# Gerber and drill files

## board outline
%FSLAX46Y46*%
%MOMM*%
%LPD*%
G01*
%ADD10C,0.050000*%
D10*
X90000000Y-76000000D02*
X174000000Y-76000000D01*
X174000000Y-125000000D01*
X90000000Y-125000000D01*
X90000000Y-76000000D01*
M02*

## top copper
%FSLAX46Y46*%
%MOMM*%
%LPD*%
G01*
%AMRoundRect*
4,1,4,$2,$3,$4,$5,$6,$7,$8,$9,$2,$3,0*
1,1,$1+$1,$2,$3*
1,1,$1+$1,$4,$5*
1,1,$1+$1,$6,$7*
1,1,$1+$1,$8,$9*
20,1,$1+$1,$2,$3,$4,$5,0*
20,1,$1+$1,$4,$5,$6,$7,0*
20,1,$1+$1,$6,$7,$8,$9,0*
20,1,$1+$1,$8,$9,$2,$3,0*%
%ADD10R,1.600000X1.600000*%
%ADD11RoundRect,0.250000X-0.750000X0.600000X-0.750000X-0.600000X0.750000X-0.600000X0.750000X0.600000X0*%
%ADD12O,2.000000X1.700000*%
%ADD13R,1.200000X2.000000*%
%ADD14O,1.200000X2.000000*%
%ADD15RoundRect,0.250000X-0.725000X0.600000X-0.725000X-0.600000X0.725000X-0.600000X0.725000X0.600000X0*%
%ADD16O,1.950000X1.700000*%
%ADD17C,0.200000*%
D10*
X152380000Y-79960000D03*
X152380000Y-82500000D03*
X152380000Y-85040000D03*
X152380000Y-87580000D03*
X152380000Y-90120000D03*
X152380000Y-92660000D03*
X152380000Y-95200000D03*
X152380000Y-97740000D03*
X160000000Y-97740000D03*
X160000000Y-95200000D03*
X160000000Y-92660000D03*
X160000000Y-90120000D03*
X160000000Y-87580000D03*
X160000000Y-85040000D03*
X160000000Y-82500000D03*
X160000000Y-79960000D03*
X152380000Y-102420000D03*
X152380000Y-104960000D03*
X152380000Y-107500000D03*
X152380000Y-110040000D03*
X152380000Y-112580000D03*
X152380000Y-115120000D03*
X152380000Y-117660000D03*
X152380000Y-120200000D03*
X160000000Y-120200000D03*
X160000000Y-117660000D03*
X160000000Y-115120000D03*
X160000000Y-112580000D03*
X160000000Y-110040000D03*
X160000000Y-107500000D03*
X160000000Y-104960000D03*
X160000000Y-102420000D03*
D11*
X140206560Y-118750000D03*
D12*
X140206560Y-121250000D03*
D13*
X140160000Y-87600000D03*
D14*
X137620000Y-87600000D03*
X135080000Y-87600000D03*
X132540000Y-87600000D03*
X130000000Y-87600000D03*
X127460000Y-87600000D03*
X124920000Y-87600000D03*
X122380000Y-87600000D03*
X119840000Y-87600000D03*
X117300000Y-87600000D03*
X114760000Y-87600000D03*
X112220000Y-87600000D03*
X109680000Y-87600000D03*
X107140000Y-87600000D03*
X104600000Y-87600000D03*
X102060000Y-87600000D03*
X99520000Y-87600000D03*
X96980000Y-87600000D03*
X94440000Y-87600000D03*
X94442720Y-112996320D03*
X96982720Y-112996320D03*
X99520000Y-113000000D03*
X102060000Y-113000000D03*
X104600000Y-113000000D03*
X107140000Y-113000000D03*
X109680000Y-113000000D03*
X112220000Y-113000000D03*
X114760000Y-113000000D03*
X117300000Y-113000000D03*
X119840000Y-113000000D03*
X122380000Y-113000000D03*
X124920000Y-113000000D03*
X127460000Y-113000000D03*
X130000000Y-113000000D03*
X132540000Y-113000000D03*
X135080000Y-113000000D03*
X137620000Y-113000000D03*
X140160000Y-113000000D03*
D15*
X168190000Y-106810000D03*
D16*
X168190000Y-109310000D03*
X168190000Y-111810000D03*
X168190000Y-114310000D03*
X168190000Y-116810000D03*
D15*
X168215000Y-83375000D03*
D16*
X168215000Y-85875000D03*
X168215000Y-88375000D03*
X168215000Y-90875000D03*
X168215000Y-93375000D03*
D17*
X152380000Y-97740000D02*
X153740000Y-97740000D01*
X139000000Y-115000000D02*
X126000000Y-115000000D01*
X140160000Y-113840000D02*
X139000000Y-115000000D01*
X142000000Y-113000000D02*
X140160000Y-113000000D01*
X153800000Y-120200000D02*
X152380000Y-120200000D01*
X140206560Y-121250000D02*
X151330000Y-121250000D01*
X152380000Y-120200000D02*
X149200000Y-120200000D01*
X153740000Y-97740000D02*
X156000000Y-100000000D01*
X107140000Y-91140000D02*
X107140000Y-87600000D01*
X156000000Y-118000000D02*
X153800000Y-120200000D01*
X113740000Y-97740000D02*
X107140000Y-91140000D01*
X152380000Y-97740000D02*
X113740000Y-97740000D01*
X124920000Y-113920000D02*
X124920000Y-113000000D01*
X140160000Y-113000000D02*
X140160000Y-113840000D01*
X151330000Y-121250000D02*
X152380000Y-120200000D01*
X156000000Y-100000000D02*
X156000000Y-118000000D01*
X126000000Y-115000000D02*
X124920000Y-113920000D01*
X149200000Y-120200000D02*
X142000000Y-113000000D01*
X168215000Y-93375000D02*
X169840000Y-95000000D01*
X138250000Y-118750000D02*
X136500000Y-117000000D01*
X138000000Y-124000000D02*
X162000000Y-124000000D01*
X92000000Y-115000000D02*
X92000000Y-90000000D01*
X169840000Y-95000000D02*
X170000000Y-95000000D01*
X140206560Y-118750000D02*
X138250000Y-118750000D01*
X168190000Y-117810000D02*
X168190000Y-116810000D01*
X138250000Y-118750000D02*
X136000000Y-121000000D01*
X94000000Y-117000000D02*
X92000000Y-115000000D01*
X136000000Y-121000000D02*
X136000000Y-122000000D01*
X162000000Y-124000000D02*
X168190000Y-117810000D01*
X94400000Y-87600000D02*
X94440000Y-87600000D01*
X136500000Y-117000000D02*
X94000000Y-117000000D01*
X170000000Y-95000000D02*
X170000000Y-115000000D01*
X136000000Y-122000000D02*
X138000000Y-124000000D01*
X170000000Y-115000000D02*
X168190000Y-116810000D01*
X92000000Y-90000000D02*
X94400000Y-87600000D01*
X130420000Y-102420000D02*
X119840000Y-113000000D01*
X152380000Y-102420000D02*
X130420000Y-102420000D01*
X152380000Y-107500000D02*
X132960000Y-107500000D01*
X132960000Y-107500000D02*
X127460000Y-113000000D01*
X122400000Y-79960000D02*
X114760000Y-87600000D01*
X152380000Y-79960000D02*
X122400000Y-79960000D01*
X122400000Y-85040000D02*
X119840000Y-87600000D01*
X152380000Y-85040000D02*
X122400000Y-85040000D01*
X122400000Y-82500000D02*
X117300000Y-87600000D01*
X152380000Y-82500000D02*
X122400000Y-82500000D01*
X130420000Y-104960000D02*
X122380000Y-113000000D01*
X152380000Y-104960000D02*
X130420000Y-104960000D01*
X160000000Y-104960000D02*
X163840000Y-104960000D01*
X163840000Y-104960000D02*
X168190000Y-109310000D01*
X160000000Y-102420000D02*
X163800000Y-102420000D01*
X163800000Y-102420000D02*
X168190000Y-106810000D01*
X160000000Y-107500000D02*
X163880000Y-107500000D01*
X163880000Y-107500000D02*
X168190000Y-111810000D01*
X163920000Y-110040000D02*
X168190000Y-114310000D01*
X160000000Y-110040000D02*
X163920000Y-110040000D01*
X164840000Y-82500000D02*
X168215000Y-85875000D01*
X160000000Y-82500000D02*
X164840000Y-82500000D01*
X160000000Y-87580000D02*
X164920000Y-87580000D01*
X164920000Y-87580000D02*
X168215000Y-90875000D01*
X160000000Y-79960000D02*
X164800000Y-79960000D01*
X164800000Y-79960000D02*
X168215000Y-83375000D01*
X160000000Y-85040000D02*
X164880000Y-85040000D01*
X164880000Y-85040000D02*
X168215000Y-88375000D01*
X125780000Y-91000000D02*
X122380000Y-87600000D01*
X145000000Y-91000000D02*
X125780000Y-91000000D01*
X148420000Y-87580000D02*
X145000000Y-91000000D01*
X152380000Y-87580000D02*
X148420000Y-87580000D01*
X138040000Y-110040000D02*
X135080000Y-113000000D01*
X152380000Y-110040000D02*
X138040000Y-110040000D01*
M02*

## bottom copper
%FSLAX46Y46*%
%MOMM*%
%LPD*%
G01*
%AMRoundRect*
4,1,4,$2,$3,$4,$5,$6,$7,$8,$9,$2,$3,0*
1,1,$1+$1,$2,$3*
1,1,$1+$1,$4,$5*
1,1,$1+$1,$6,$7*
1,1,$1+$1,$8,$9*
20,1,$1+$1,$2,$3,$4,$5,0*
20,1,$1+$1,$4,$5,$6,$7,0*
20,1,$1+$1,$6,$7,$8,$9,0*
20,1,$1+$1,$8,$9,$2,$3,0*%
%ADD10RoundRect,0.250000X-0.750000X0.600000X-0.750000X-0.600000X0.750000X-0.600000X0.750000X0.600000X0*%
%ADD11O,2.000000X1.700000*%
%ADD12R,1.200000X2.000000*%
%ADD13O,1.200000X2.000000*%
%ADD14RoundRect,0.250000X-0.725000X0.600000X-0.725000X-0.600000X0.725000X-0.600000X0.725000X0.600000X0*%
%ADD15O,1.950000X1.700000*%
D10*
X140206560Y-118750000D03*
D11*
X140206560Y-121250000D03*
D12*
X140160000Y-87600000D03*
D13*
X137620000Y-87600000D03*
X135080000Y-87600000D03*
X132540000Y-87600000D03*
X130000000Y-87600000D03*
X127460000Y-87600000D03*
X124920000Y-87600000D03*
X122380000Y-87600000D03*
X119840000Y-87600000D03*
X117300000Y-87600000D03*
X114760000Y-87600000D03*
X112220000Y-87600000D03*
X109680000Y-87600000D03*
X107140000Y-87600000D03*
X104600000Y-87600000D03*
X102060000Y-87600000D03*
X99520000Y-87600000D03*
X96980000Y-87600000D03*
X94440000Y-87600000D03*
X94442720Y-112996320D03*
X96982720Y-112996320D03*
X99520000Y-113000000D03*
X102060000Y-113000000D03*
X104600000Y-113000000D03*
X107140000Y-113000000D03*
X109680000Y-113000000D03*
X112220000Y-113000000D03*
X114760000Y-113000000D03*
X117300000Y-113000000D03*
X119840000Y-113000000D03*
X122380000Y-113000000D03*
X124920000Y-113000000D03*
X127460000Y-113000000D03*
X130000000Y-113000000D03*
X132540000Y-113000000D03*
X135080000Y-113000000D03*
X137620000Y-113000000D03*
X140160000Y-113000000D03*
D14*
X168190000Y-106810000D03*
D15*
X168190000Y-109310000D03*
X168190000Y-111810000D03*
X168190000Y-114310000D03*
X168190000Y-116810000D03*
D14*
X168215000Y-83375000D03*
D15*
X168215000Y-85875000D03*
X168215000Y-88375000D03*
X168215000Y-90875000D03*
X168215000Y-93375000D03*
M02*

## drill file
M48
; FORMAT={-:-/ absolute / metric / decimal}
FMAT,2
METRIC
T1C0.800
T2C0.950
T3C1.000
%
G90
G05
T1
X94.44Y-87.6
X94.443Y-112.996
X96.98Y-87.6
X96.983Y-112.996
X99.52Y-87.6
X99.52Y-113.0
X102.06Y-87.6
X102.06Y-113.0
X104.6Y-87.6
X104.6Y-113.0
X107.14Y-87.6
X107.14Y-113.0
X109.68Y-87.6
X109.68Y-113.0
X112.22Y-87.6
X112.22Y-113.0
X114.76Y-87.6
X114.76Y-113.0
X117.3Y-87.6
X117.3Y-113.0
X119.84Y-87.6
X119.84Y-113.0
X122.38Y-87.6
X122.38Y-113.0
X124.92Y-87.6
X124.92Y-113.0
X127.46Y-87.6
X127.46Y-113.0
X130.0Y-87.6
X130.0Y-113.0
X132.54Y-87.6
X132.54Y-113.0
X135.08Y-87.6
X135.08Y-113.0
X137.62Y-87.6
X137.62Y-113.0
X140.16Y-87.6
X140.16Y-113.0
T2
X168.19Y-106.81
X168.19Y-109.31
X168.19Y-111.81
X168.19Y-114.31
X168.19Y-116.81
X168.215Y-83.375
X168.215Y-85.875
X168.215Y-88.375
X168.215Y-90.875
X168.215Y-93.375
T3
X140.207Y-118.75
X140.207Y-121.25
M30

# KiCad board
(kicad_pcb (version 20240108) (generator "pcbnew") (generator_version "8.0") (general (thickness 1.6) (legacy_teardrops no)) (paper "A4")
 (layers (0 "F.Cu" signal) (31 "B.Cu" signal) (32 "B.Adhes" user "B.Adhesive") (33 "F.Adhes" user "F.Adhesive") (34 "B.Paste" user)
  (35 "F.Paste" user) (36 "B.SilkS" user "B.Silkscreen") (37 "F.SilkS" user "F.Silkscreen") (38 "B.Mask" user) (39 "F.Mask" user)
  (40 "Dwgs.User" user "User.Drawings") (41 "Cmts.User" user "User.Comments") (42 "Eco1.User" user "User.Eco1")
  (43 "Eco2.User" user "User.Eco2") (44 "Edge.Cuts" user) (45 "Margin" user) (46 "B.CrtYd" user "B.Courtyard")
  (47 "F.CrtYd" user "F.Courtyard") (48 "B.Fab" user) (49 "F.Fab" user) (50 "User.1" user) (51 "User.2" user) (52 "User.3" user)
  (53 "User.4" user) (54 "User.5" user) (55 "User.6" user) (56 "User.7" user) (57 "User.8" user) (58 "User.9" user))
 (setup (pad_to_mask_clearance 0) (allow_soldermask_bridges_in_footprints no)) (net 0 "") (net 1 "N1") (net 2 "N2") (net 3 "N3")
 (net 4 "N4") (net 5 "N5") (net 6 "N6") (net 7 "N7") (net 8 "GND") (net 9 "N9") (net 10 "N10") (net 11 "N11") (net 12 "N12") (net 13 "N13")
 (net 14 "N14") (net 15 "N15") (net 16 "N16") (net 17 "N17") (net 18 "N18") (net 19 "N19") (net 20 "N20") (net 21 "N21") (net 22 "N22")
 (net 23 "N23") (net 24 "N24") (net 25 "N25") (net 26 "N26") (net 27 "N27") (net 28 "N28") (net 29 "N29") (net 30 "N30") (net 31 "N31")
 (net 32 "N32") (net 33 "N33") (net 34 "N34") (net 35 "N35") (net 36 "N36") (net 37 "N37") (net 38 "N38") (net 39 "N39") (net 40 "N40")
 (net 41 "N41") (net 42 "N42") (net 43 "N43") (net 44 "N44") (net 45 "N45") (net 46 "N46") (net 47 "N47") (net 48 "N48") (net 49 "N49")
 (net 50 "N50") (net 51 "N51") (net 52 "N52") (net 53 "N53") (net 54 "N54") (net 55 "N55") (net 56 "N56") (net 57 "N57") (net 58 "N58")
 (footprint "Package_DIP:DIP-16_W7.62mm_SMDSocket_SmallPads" (layer "F.Cu") (at 156.19 88.85)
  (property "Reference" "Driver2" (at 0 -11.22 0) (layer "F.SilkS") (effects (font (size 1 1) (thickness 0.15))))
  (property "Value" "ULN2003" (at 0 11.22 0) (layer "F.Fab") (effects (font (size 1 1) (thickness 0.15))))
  (pad "1" smd rect (at -3.81 -8.89) (size 1.6 1.6) (layers "F.Cu" "F.Paste" "F.Mask") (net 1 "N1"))
  (pad "2" smd rect (at -3.81 -6.35) (size 1.6 1.6) (layers "F.Cu" "F.Paste" "F.Mask") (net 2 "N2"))
  (pad "3" smd rect (at -3.81 -3.81) (size 1.6 1.6) (layers "F.Cu" "F.Paste" "F.Mask") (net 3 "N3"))
  (pad "4" smd rect (at -3.81 -1.27) (size 1.6 1.6) (layers "F.Cu" "F.Paste" "F.Mask") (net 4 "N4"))
  (pad "5" smd rect (at -3.81 1.27) (size 1.6 1.6) (layers "F.Cu" "F.Paste" "F.Mask") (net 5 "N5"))
  (pad "6" smd rect (at -3.81 3.81) (size 1.6 1.6) (layers "F.Cu" "F.Paste" "F.Mask") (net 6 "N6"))
  (pad "7" smd rect (at -3.81 6.35) (size 1.6 1.6) (layers "F.Cu" "F.Paste" "F.Mask") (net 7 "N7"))
  (pad "8" smd rect (at -3.81 8.89) (size 1.6 1.6) (layers "F.Cu" "F.Paste" "F.Mask") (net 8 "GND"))
  (pad "9" smd rect (at 3.81 8.89) (size 1.6 1.6) (layers "F.Cu" "F.Paste" "F.Mask") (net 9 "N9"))
  (pad "10" smd rect (at 3.81 6.35) (size 1.6 1.6) (layers "F.Cu" "F.Paste" "F.Mask") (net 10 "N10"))
  (pad "11" smd rect (at 3.81 3.81) (size 1.6 1.6) (layers "F.Cu" "F.Paste" "F.Mask") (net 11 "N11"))
  (pad "12" smd rect (at 3.81 1.27) (size 1.6 1.6) (layers "F.Cu" "F.Paste" "F.Mask") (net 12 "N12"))
  (pad "13" smd rect (at 3.81 -1.27) (size 1.6 1.6) (layers "F.Cu" "F.Paste" "F.Mask") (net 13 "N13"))
  (pad "14" smd rect (at 3.81 -3.81) (size 1.6 1.6) (layers "F.Cu" "F.Paste" "F.Mask") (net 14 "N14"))
  (pad "15" smd rect (at 3.81 -6.35) (size 1.6 1.6) (layers "F.Cu" "F.Paste" "F.Mask") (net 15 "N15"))
  (pad "16" smd rect (at 3.81 -8.89) (size 1.6 1.6) (layers "F.Cu" "F.Paste" "F.Mask") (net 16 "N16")))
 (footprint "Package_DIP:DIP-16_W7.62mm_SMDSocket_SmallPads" (layer "F.Cu") (at 156.19 111.31)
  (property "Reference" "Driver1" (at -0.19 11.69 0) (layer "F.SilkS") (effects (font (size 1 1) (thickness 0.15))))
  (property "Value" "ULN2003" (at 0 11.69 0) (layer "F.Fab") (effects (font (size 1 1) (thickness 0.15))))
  (pad "1" smd rect (at -3.81 -8.89) (size 1.6 1.6) (layers "F.Cu" "F.Paste" "F.Mask") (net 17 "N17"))
  (pad "2" smd rect (at -3.81 -6.35) (size 1.6 1.6) (layers "F.Cu" "F.Paste" "F.Mask") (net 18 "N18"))
  (pad "3" smd rect (at -3.81 -3.81) (size 1.6 1.6) (layers "F.Cu" "F.Paste" "F.Mask") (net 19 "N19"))
  (pad "4" smd rect (at -3.81 -1.27) (size 1.6 1.6) (layers "F.Cu" "F.Paste" "F.Mask") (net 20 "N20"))
  (pad "5" smd rect (at -3.81 1.27) (size 1.6 1.6) (layers "F.Cu" "F.Paste" "F.Mask") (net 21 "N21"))
  (pad "6" smd rect (at -3.81 3.81) (size 1.6 1.6) (layers "F.Cu" "F.Paste" "F.Mask") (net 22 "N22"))
  (pad "7" smd rect (at -3.81 6.35) (size 1.6 1.6) (layers "F.Cu" "F.Paste" "F.Mask") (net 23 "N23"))
  (pad "8" smd rect (at -3.81 8.89) (size 1.6 1.6) (layers "F.Cu" "F.Paste" "F.Mask") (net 8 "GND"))
  (pad "9" smd rect (at 3.81 8.89) (size 1.6 1.6) (layers "F.Cu" "F.Paste" "F.Mask") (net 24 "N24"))
  (pad "10" smd rect (at 3.81 6.35) (size 1.6 1.6) (layers "F.Cu" "F.Paste" "F.Mask") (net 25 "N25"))
  (pad "11" smd rect (at 3.81 3.81) (size 1.6 1.6) (layers "F.Cu" "F.Paste" "F.Mask") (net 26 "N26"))
  (pad "12" smd rect (at 3.81 1.27) (size 1.6 1.6) (layers "F.Cu" "F.Paste" "F.Mask") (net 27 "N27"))
  (pad "13" smd rect (at 3.81 -1.27) (size 1.6 1.6) (layers "F.Cu" "F.Paste" "F.Mask") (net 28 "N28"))
  (pad "14" smd rect (at 3.81 -3.81) (size 1.6 1.6) (layers "F.Cu" "F.Paste" "F.Mask") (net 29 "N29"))
  (pad "15" smd rect (at 3.81 -6.35) (size 1.6 1.6) (layers "F.Cu" "F.Paste" "F.Mask") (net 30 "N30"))
  (pad "16" smd rect (at 3.81 -8.89) (size 1.6 1.6) (layers "F.Cu" "F.Paste" "F.Mask") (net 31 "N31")))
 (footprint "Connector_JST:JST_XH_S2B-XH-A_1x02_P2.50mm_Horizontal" (layer "F.Cu") (at 140.20656 118.75 -90)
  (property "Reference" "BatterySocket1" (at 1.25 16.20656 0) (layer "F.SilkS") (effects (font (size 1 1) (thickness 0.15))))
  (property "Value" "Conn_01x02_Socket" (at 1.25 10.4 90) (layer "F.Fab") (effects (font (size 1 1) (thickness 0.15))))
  (pad "1" thru_hole roundrect (at 0 0 270) (size 1.7 2) (drill 1) (layers "*.Cu" "*.Mask") (remove_unused_layers no)
   (roundrect_rratio 0.147059) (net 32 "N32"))
  (pad "2" thru_hole oval (at 2.5 0 270) (size 1.7 2) (drill 1) (layers "*.Cu" "*.Mask") (remove_unused_layers no) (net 8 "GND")))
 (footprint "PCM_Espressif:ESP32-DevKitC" (layer "F.Cu") (at 140.16 87.6 -90)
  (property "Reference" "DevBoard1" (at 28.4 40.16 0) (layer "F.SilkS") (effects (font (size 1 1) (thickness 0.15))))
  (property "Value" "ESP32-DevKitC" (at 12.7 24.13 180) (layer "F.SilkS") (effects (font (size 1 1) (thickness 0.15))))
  (pad "1" thru_hole rect (at 0 0 180) (size 1.2 2) (drill 0.8) (layers "*.Cu" "*.Mask") (remove_unused_layers no) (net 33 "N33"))
  (pad "2" thru_hole oval (at 0 2.54 180) (size 1.2 2) (drill 0.8) (layers "*.Cu" "*.Mask") (remove_unused_layers no) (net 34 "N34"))
  (pad "3" thru_hole oval (at 0 5.08 180) (size 1.2 2) (drill 0.8) (layers "*.Cu" "*.Mask") (remove_unused_layers no) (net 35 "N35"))
  (pad "4" thru_hole oval (at 0 7.62 180) (size 1.2 2) (drill 0.8) (layers "*.Cu" "*.Mask") (remove_unused_layers no) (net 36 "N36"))
  (pad "5" thru_hole oval (at 0 10.16 180) (size 1.2 2) (drill 0.8) (layers "*.Cu" "*.Mask") (remove_unused_layers no) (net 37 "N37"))
  (pad "6" thru_hole oval (at 0 12.7 180) (size 1.2 2) (drill 0.8) (layers "*.Cu" "*.Mask") (remove_unused_layers no) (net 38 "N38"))
  (pad "7" thru_hole oval (at 0 15.24 180) (size 1.2 2) (drill 0.8) (layers "*.Cu" "*.Mask") (remove_unused_layers no) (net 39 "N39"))
  (pad "8" thru_hole oval (at 0 17.78 180) (size 1.2 2) (drill 0.8) (layers "*.Cu" "*.Mask") (remove_unused_layers no) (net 4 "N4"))
  (pad "9" thru_hole oval (at 0 20.32 180) (size 1.2 2) (drill 0.8) (layers "*.Cu" "*.Mask") (remove_unused_layers no) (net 3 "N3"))
  (pad "10" thru_hole oval (at 0 22.86 180) (size 1.2 2) (drill 0.8) (layers "*.Cu" "*.Mask") (remove_unused_layers no) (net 2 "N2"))
  (pad "11" thru_hole oval (at 0 25.4 180) (size 1.2 2) (drill 0.8) (layers "*.Cu" "*.Mask") (remove_unused_layers no) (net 1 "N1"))
  (pad "12" thru_hole oval (at 0 27.94 180) (size 1.2 2) (drill 0.8) (layers "*.Cu" "*.Mask") (remove_unused_layers no) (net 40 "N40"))
  (pad "13" thru_hole oval (at 0 30.48 180) (size 1.2 2) (drill 0.8) (layers "*.Cu" "*.Mask") (remove_unused_layers no) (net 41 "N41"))
  (pad "14" thru_hole oval (at 0 33.02 180) (size 1.2 2) (drill 0.8) (layers "*.Cu" "*.Mask") (remove_unused_layers no) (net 8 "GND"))
  (pad "15" thru_hole oval (at 0 35.56 180) (size 1.2 2) (drill 0.8) (layers "*.Cu" "*.Mask") (remove_unused_layers no) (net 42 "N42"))
  (pad "16" thru_hole oval (at 0 38.1 180) (size 1.2 2) (drill 0.8) (layers "*.Cu" "*.Mask") (remove_unused_layers no) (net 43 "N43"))
  (pad "17" thru_hole oval (at 0 40.64 180) (size 1.2 2) (drill 0.8) (layers "*.Cu" "*.Mask") (remove_unused_layers no) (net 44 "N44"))
  (pad "18" thru_hole oval (at 0 43.18 180) (size 1.2 2) (drill 0.8) (layers "*.Cu" "*.Mask") (remove_unused_layers no) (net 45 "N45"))
  (pad "19" thru_hole oval (at 0 45.72 180) (size 1.2 2) (drill 0.8) (layers "*.Cu" "*.Mask") (remove_unused_layers no) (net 32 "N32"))
  (pad "20" thru_hole oval (at 25.39632 45.71728 180) (size 1.2 2) (drill 0.8) (layers "*.Cu" "*.Mask") (remove_unused_layers no)
   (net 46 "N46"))
  (pad "21" thru_hole oval (at 25.39632 43.17728 180) (size 1.2 2) (drill 0.8) (layers "*.Cu" "*.Mask") (remove_unused_layers no)
   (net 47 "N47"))
  (pad "22" thru_hole oval (at 25.4 40.64 180) (size 1.2 2) (drill 0.8) (layers "*.Cu" "*.Mask") (remove_unused_layers no) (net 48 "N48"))
  (pad "23" thru_hole oval (at 25.4 38.1 180) (size 1.2 2) (drill 0.8) (layers "*.Cu" "*.Mask") (remove_unused_layers no) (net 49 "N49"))
  (pad "24" thru_hole oval (at 25.4 35.56 180) (size 1.2 2) (drill 0.8) (layers "*.Cu" "*.Mask") (remove_unused_layers no) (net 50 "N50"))
  (pad "25" thru_hole oval (at 25.4 33.02 180) (size 1.2 2) (drill 0.8) (layers "*.Cu" "*.Mask") (remove_unused_layers no) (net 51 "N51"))
  (pad "26" thru_hole oval (at 25.4 30.48 180) (size 1.2 2) (drill 0.8) (layers "*.Cu" "*.Mask") (remove_unused_layers no) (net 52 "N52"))
  (pad "27" thru_hole oval (at 25.4 27.94 180) (size 1.2 2) (drill 0.8) (layers "*.Cu" "*.Mask") (remove_unused_layers no) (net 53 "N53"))
  (pad "28" thru_hole oval (at 25.4 25.4 180) (size 1.2 2) (drill 0.8) (layers "*.Cu" "*.Mask") (remove_unused_layers no) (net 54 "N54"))
  (pad "29" thru_hole oval (at 25.4 22.86 180) (size 1.2 2) (drill 0.8) (layers "*.Cu" "*.Mask") (remove_unused_layers no) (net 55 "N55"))
  (pad "30" thru_hole oval (at 25.4 20.32 180) (size 1.2 2) (drill 0.8) (layers "*.Cu" "*.Mask") (remove_unused_layers no) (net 17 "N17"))
  (pad "31" thru_hole oval (at 25.4 17.78 180) (size 1.2 2) (drill 0.8) (layers "*.Cu" "*.Mask") (remove_unused_layers no) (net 18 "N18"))
  (pad "32" thru_hole oval (at 25.4 15.24 180) (size 1.2 2) (drill 0.8) (layers "*.Cu" "*.Mask") (remove_unused_layers no) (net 8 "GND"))
  (pad "33" thru_hole oval (at 25.4 12.7 180) (size 1.2 2) (drill 0.8) (layers "*.Cu" "*.Mask") (remove_unused_layers no) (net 19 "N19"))
  (pad "34" thru_hole oval (at 25.4 10.16 180) (size 1.2 2) (drill 0.8) (layers "*.Cu" "*.Mask") (remove_unused_layers no) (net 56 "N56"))
  (pad "35" thru_hole oval (at 25.4 7.62 180) (size 1.2 2) (drill 0.8) (layers "*.Cu" "*.Mask") (remove_unused_layers no) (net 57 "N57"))
  (pad "36" thru_hole oval (at 25.4 5.08 180) (size 1.2 2) (drill 0.8) (layers "*.Cu" "*.Mask") (remove_unused_layers no) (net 20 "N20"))
  (pad "37" thru_hole oval (at 25.4 2.54 180) (size 1.2 2) (drill 0.8) (layers "*.Cu" "*.Mask") (remove_unused_layers no) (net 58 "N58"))
  (pad "38" thru_hole oval (at 25.4 0 180) (size 1.2 2) (drill 0.8) (layers "*.Cu" "*.Mask") (remove_unused_layers no) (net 8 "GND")))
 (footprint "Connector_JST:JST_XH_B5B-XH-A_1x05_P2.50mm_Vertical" (layer "F.Cu") (at 168.19 106.81 -90)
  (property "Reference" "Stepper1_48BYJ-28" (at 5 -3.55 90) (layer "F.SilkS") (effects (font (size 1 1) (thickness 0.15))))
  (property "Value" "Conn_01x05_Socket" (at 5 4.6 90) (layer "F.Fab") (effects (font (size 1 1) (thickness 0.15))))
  (pad "1" thru_hole roundrect (at 0 0 270) (size 1.7 1.95) (drill 0.95) (layers "*.Cu" "*.Mask") (remove_unused_layers no)
   (roundrect_rratio 0.147059) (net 31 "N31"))
  (pad "2" thru_hole oval (at 2.5 0 270) (size 1.7 1.95) (drill 0.95) (layers "*.Cu" "*.Mask") (remove_unused_layers no) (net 30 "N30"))
  (pad "3" thru_hole oval (at 5 0 270) (size 1.7 1.95) (drill 0.95) (layers "*.Cu" "*.Mask") (remove_unused_layers no) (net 29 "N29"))
  (pad "4" thru_hole oval (at 7.5 0 270) (size 1.7 1.95) (drill 0.95) (layers "*.Cu" "*.Mask") (remove_unused_layers no) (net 28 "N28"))
  (pad "5" thru_hole oval (at 10 0 270) (size 1.7 1.95) (drill 0.95) (layers "*.Cu" "*.Mask") (remove_unused_layers no) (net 32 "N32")))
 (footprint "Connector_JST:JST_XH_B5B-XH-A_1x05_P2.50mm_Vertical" (layer "F.Cu") (at 168.215 83.375 -90)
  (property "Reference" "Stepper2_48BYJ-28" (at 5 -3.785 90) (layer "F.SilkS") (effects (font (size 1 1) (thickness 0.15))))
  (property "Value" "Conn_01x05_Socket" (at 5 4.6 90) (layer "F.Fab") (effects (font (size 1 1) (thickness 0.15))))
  (pad "1" thru_hole roundrect (at 0 0 270) (size 1.7 1.95) (drill 0.95) (layers "*.Cu" "*.Mask") (remove_unused_layers no)
   (roundrect_rratio 0.147059) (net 16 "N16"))
  (pad "2" thru_hole oval (at 2.5 0 270) (size 1.7 1.95) (drill 0.95) (layers "*.Cu" "*.Mask") (remove_unused_layers no) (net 15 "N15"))
  (pad "3" thru_hole oval (at 5 0 270) (size 1.7 1.95) (drill 0.95) (layers "*.Cu" "*.Mask") (remove_unused_layers no) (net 14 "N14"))
  (pad "4" thru_hole oval (at 7.5 0 270) (size 1.7 1.95) (drill 0.95) (layers "*.Cu" "*.Mask") (remove_unused_layers no) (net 13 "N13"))
  (pad "5" thru_hole oval (at 10 0 270) (size 1.7 1.95) (drill 0.95) (layers "*.Cu" "*.Mask") (remove_unused_layers no) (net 32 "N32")))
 (gr_rect (start 90 76) (end 174 125) (stroke (width 0.05) (type default)) (fill none) (layer "Edge.Cuts"))
 (segment (start 152.38 97.74) (end 153.74 97.74) (width 0.2) (layer "F.Cu") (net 8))
 (segment (start 139 115) (end 126 115) (width 0.2) (layer "F.Cu") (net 8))
 (segment (start 140.16 113.84) (end 139 115) (width 0.2) (layer "F.Cu") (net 8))
 (segment (start 142 113) (end 140.16 113) (width 0.2) (layer "F.Cu") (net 8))
 (segment (start 153.8 120.2) (end 152.38 120.2) (width 0.2) (layer "F.Cu") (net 8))
 (segment (start 140.20656 121.25) (end 151.33 121.25) (width 0.2) (layer "F.Cu") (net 8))
 (segment (start 152.38 120.2) (end 149.2 120.2) (width 0.2) (layer "F.Cu") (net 8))
 (segment (start 153.74 97.74) (end 156 100) (width 0.2) (layer "F.Cu") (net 8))
 (segment (start 107.14 91.14) (end 107.14 87.6) (width 0.2) (layer "F.Cu") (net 8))
 (segment (start 156 118) (end 153.8 120.2) (width 0.2) (layer "F.Cu") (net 8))
 (segment (start 113.74 97.74) (end 107.14 91.14) (width 0.2) (layer "F.Cu") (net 8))
 (segment (start 152.38 97.74) (end 113.74 97.74) (width 0.2) (layer "F.Cu") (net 8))
 (segment (start 124.92 113.92) (end 124.92 113) (width 0.2) (layer "F.Cu") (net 8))
 (segment (start 140.16 113) (end 140.16 113.84) (width 0.2) (layer "F.Cu") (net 8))
 (segment (start 151.33 121.25) (end 152.38 120.2) (width 0.2) (layer "F.Cu") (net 8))
 (segment (start 156 100) (end 156 118) (width 0.2) (layer "F.Cu") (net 8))
 (segment (start 126 115) (end 124.92 113.92) (width 0.2) (layer "F.Cu") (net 8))
 (segment (start 149.2 120.2) (end 142 113) (width 0.2) (layer "F.Cu") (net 8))
 (segment (start 168.215 93.375) (end 169.84 95) (width 0.2) (layer "F.Cu") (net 32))
 (segment (start 138.25 118.75) (end 136.5 117) (width 0.2) (layer "F.Cu") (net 32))
 (segment (start 138 124) (end 162 124) (width 0.2) (layer "F.Cu") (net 32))
 (segment (start 92 115) (end 92 90) (width 0.2) (layer "F.Cu") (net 32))
 (segment (start 169.84 95) (end 170 95) (width 0.2) (layer "F.Cu") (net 32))
 (segment (start 140.20656 118.75) (end 138.25 118.75) (width 0.2) (layer "F.Cu") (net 32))
 (segment (start 168.19 117.81) (end 168.19 116.81) (width 0.2) (layer "F.Cu") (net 32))
 (segment (start 138.25 118.75) (end 136 121) (width 0.2) (layer "F.Cu") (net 32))
 (segment (start 94 117) (end 92 115) (width 0.2) (layer "F.Cu") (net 32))
 (segment (start 136 121) (end 136 122) (width 0.2) (layer "F.Cu") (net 32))
 (segment (start 162 124) (end 168.19 117.81) (width 0.2) (layer "F.Cu") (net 32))
 (segment (start 94.4 87.6) (end 94.44 87.6) (width 0.2) (layer "F.Cu") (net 32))
 (segment (start 136.5 117) (end 94 117) (width 0.2) (layer "F.Cu") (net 32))
 (segment (start 170 95) (end 170 115) (width 0.2) (layer "F.Cu") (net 32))
 (segment (start 136 122) (end 138 124) (width 0.2) (layer "F.Cu") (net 32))
 (segment (start 170 115) (end 168.19 116.81) (width 0.2) (layer "F.Cu") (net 32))
 (segment (start 92 90) (end 94.4 87.6) (width 0.2) (layer "F.Cu") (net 32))
 (segment (start 130.42 102.42) (end 119.84 113) (width 0.2) (layer "F.Cu") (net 17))
 (segment (start 152.38 102.42) (end 130.42 102.42) (width 0.2) (layer "F.Cu") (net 17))
 (segment (start 152.38 107.5) (end 132.96 107.5) (width 0.2) (layer "F.Cu") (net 19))
 (segment (start 132.96 107.5) (end 127.46 113) (width 0.2) (layer "F.Cu") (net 19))
 (segment (start 122.4 79.96) (end 114.76 87.6) (width 0.2) (layer "F.Cu") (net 1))
 (segment (start 152.38 79.96) (end 122.4 79.96) (width 0.2) (layer "F.Cu") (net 1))
 (segment (start 122.4 85.04) (end 119.84 87.6) (width 0.2) (layer "F.Cu") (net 3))
 (segment (start 152.38 85.04) (end 122.4 85.04) (width 0.2) (layer "F.Cu") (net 3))
 (segment (start 122.4 82.5) (end 117.3 87.6) (width 0.2) (layer "F.Cu") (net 2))
 (segment (start 152.38 82.5) (end 122.4 82.5) (width 0.2) (layer "F.Cu") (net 2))
 (segment (start 130.42 104.96) (end 122.38 113) (width 0.2) (layer "F.Cu") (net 18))
 (segment (start 152.38 104.96) (end 130.42 104.96) (width 0.2) (layer "F.Cu") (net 18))
 (segment (start 160 104.96) (end 163.84 104.96) (width 0.2) (layer "F.Cu") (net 30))
 (segment (start 163.84 104.96) (end 168.19 109.31) (width 0.2) (layer "F.Cu") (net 30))
 (segment (start 160 102.42) (end 163.8 102.42) (width 0.2) (layer "F.Cu") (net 31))
 (segment (start 163.8 102.42) (end 168.19 106.81) (width 0.2) (layer "F.Cu") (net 31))
 (segment (start 160 107.5) (end 163.88 107.5) (width 0.2) (layer "F.Cu") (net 29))
 (segment (start 163.88 107.5) (end 168.19 111.81) (width 0.2) (layer "F.Cu") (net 29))
 (segment (start 163.92 110.04) (end 168.19 114.31) (width 0.2) (layer "F.Cu") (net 28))
 (segment (start 160 110.04) (end 163.92 110.04) (width 0.2) (layer "F.Cu") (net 28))
 (segment (start 164.84 82.5) (end 168.215 85.875) (width 0.2) (layer "F.Cu") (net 15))
 (segment (start 160 82.5) (end 164.84 82.5) (width 0.2) (layer "F.Cu") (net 15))
 (segment (start 160 87.58) (end 164.92 87.58) (width 0.2) (layer "F.Cu") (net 13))
 (segment (start 164.92 87.58) (end 168.215 90.875) (width 0.2) (layer "F.Cu") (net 13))
 (segment (start 160 79.96) (end 164.8 79.96) (width 0.2) (layer "F.Cu") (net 16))
 (segment (start 164.8 79.96) (end 168.215 83.375) (width 0.2) (layer "F.Cu") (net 16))
 (segment (start 160 85.04) (end 164.88 85.04) (width 0.2) (layer "F.Cu") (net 14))
 (segment (start 164.88 85.04) (end 168.215 88.375) (width 0.2) (layer "F.Cu") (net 14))
 (segment (start 125.78 91) (end 122.38 87.6) (width 0.2) (layer "F.Cu") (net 4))
 (segment (start 145 91) (end 125.78 91) (width 0.2) (layer "F.Cu") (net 4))
 (segment (start 148.42 87.58) (end 145 91) (width 0.2) (layer "F.Cu") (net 4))
 (segment (start 152.38 87.58) (end 148.42 87.58) (width 0.2) (layer "F.Cu") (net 4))
 (segment (start 138.04 110.04) (end 135.08 113) (width 0.2) (layer "F.Cu") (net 20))
 (segment (start 152.38 110.04) (end 138.04 110.04) (width 0.2) (layer "F.Cu") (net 20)))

